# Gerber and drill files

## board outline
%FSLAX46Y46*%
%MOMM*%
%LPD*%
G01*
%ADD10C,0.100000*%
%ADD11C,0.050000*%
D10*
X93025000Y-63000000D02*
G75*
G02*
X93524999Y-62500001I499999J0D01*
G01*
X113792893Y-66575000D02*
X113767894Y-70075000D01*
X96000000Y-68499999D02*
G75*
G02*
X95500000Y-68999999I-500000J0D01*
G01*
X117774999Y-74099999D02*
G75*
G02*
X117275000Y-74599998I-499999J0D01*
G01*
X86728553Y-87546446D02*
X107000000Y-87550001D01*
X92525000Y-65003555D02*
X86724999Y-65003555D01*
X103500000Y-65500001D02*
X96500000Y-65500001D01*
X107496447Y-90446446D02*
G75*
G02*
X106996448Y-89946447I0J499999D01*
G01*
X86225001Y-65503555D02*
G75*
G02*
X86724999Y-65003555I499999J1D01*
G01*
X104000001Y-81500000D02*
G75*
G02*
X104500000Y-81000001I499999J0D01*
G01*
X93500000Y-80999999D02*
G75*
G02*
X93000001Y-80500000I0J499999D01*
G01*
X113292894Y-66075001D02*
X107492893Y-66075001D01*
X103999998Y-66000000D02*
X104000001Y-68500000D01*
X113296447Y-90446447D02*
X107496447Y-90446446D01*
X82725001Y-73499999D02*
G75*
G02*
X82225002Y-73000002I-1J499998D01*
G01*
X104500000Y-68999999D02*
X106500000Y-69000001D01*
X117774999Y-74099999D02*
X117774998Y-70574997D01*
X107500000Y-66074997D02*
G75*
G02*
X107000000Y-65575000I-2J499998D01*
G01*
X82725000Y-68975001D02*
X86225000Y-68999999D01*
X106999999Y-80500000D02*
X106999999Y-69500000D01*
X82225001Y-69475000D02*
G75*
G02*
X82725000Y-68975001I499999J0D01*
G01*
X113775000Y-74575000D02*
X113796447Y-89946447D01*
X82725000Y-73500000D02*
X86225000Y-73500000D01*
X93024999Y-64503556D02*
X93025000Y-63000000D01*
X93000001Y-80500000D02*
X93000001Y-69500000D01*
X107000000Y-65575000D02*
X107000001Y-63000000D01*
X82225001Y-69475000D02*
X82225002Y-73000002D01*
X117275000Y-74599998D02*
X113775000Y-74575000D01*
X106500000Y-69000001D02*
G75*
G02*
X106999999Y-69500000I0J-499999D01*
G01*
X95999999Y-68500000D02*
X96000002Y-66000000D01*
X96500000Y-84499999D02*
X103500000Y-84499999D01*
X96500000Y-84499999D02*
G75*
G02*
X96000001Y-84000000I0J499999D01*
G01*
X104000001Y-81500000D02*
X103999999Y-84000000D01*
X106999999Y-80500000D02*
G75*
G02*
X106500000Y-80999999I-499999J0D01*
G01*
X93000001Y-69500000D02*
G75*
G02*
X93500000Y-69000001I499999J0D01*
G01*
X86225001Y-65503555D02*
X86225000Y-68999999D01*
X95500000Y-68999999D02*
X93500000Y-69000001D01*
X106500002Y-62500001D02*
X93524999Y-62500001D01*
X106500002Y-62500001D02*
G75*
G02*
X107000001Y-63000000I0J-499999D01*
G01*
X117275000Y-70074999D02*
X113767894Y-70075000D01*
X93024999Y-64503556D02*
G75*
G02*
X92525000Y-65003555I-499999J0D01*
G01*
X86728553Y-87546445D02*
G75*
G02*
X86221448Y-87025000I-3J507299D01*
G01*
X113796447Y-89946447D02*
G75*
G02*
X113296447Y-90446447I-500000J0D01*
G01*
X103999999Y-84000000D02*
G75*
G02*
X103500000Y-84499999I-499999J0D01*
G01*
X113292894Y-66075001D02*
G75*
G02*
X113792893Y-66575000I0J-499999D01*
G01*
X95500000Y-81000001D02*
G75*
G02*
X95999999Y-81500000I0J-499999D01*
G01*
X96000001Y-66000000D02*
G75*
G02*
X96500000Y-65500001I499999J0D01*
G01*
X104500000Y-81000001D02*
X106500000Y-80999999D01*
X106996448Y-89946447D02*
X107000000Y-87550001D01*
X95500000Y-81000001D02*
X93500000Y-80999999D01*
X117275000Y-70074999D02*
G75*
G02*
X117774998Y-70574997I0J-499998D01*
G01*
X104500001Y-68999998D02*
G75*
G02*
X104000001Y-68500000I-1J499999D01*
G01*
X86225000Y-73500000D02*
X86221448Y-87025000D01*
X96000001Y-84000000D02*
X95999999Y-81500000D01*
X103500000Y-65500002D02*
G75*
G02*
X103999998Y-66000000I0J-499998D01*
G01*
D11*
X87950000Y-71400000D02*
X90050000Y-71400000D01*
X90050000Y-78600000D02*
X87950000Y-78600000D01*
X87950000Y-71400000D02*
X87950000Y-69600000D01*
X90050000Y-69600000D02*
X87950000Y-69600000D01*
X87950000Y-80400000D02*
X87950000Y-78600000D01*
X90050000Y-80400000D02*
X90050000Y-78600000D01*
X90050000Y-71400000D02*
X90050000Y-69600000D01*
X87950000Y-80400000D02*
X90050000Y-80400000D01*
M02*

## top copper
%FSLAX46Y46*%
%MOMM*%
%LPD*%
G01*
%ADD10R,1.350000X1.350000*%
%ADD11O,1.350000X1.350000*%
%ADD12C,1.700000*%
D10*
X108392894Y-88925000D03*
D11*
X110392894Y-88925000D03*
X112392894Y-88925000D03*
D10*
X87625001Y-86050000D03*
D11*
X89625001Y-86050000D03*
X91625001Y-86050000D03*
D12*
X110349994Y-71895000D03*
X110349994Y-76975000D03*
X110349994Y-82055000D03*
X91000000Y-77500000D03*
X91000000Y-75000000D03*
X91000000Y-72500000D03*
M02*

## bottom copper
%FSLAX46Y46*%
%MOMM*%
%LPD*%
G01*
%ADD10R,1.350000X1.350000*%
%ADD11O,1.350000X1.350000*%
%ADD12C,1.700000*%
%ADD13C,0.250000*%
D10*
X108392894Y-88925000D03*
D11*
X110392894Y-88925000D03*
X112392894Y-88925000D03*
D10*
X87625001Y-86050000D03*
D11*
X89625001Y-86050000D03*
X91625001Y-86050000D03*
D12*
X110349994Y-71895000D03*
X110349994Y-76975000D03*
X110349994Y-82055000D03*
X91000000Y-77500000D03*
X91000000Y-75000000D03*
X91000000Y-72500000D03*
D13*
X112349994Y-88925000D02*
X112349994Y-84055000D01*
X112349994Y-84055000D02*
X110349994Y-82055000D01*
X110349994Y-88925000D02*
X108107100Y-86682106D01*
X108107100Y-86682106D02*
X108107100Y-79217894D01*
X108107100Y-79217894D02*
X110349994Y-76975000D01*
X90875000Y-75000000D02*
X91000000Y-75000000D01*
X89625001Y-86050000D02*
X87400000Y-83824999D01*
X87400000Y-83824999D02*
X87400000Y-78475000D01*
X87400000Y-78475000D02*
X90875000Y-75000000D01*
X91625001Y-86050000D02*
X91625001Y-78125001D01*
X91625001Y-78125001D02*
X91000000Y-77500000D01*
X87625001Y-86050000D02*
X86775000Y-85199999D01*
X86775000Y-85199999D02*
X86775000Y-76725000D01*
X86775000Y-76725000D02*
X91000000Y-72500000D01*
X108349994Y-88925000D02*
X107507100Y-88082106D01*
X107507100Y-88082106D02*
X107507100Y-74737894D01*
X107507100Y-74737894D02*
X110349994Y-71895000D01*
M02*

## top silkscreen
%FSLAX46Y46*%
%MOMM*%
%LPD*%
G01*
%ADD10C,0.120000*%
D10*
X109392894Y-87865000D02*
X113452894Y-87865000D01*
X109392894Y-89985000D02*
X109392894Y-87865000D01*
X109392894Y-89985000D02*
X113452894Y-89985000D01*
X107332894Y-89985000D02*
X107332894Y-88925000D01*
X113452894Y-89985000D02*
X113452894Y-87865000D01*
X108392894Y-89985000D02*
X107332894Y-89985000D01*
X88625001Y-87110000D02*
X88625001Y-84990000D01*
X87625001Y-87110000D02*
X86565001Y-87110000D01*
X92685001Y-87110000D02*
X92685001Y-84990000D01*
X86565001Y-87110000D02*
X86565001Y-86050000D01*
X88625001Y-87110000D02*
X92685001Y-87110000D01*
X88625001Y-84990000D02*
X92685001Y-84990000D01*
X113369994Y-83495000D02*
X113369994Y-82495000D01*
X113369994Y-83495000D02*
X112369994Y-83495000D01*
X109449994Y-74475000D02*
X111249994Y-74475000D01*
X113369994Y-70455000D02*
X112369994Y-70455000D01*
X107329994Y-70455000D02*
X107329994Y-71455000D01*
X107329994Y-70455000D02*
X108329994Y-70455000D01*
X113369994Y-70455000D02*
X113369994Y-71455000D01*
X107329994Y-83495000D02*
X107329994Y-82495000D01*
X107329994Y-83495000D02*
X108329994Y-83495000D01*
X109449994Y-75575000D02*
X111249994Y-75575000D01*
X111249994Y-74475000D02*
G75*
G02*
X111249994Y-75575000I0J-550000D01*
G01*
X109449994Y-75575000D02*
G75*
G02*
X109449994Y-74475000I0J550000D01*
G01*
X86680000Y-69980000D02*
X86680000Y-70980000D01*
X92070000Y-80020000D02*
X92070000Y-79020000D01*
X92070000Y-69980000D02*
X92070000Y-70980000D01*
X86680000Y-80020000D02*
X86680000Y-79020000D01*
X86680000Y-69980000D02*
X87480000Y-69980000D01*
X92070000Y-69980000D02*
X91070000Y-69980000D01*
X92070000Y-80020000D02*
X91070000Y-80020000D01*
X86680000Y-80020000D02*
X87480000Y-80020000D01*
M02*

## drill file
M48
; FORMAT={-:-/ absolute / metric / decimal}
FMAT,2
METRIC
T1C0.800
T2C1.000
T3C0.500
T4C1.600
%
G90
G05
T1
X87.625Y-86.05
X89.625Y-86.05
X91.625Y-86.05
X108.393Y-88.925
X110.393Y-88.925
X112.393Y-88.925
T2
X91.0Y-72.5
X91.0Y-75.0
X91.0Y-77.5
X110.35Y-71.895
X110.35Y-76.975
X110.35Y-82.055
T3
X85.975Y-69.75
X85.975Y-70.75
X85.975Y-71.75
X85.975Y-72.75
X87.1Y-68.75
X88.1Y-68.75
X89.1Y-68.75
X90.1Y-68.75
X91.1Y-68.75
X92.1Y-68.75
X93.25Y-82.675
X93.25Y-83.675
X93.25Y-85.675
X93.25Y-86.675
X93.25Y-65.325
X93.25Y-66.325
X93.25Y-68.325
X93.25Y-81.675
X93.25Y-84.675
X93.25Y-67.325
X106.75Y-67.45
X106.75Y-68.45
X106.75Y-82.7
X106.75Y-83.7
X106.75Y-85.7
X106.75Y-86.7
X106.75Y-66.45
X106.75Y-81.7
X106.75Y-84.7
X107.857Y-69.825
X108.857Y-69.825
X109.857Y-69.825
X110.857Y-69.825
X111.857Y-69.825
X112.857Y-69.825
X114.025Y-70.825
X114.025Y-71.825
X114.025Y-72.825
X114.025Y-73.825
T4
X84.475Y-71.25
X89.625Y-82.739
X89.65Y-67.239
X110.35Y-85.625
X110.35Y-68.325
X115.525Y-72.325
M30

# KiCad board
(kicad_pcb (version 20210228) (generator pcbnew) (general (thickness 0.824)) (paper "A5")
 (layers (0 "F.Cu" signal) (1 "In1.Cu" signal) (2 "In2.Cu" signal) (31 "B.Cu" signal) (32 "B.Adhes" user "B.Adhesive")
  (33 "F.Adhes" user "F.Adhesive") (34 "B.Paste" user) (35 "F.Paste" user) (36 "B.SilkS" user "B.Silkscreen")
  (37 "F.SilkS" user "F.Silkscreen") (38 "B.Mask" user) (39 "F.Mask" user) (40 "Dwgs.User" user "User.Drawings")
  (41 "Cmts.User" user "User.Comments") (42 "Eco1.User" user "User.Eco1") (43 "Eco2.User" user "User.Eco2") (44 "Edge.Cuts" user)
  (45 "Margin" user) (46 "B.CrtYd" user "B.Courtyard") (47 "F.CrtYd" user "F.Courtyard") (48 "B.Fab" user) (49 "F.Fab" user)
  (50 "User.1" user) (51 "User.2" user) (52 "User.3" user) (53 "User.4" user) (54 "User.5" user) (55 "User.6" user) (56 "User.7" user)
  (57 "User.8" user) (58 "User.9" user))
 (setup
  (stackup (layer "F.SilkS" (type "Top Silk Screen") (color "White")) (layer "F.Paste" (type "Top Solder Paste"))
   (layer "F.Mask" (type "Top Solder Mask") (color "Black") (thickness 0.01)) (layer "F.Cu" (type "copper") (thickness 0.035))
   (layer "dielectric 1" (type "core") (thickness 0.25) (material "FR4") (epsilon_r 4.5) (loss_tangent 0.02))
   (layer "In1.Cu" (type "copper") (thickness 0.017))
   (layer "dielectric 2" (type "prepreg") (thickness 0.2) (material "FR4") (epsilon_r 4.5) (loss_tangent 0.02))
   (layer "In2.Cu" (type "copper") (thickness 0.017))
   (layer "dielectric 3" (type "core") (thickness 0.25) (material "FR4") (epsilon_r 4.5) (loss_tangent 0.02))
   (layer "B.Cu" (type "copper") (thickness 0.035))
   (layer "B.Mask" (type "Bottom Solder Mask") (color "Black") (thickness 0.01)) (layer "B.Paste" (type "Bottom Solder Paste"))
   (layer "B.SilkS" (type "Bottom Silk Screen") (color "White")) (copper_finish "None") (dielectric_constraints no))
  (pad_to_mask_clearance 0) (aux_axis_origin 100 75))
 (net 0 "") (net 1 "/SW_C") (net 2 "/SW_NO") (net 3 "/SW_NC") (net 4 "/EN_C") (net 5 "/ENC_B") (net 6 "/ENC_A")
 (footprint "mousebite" (layer "F.Cu") (at 112.8571 69.824999 -90)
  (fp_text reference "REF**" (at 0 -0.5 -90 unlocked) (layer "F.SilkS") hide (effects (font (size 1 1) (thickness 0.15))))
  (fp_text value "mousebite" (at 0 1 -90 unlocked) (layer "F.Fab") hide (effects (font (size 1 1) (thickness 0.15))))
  (pad "" np_thru_hole circle (at 0 0 270) (size 0.5 0.5) (drill 0.5) (layers F&B.Cu *.Mask)))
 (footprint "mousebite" (layer "F.Cu") (at 93.249999 82.675001 180)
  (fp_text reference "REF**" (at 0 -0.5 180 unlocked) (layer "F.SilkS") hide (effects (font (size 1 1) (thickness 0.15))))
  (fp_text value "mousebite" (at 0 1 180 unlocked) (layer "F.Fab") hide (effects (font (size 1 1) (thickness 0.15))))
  (pad "" np_thru_hole circle (at 0 0 180) (size 0.5 0.5) (drill 0.5) (layers F&B.Cu *.Mask)))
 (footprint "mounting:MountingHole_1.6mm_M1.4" (layer "F.Cu") (at 89.650001 67.239304 -90)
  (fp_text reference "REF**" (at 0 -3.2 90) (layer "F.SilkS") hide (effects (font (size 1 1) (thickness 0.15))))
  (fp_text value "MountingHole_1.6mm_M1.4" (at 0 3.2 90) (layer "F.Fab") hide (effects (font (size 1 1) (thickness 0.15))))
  (pad "" np_thru_hole circle (at 0 0 270) (locked) (size 1.6 1.6) (drill 1.6) (layers F&B.Cu *.Mask)))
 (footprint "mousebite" (layer "F.Cu") (at 110.8571 69.824999 -90)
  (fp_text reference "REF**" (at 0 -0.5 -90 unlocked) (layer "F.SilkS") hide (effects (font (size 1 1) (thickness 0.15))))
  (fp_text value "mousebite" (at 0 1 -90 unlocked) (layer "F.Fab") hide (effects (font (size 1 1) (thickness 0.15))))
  (pad "" np_thru_hole circle (at 0 0 270) (size 0.5 0.5) (drill 0.5) (layers F&B.Cu *.Mask)))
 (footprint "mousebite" (layer "F.Cu") (at 106.749999 67.45 180)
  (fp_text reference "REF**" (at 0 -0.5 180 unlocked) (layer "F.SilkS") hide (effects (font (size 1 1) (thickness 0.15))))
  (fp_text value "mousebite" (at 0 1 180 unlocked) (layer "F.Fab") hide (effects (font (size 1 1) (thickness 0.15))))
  (pad "" np_thru_hole circle (at 0 0 180) (size 0.5 0.5) (drill 0.5) (layers F&B.Cu *.Mask)))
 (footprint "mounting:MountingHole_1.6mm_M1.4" (layer "F.Cu") (at 110.349995 68.325 -90)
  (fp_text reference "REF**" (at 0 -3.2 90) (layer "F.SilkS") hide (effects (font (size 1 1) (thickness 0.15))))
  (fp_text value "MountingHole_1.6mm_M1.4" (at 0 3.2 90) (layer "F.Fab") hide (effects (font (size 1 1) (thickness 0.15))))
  (pad "" np_thru_hole circle (at 0 0 270) (locked) (size 1.6 1.6) (drill 1.6) (layers F&B.Cu *.Mask)))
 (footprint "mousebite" (layer "F.Cu") (at 85.975 72.749998)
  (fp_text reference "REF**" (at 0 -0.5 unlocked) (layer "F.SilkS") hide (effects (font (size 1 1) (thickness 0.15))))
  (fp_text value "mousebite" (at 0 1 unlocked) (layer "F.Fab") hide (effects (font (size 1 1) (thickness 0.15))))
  (pad "" np_thru_hole circle (at 0 0) (size 0.5 0.5) (drill 0.5) (layers F&B.Cu *.Mask)))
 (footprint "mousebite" (layer "F.Cu") (at 93.249999 83.675 180)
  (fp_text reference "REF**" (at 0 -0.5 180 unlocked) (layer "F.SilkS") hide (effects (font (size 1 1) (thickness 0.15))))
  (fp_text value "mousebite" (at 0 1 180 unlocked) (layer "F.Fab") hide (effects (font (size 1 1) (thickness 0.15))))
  (pad "" np_thru_hole circle (at 0 0 180) (size 0.5 0.5) (drill 0.5) (layers F&B.Cu *.Mask)))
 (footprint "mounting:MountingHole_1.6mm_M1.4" (layer "F.Cu") (at 89.625 82.73925 -90)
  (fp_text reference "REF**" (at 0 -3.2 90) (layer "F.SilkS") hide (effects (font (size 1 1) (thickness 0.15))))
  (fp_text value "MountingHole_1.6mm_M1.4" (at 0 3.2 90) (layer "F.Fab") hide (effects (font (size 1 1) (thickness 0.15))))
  (pad "" np_thru_hole circle (at 0 0 270) (locked) (size 1.6 1.6) (drill 1.6) (layers F&B.Cu *.Mask)))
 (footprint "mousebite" (layer "F.Cu") (at 108.8571 69.824999 -90)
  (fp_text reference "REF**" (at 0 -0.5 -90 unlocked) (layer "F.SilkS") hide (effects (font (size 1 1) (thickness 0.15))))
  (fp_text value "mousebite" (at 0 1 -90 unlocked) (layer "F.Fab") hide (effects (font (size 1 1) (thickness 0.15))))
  (pad "" np_thru_hole circle (at 0 0 270) (size 0.5 0.5) (drill 0.5) (layers F&B.Cu *.Mask)))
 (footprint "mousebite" (layer "F.Cu") (at 88.1 68.75 90)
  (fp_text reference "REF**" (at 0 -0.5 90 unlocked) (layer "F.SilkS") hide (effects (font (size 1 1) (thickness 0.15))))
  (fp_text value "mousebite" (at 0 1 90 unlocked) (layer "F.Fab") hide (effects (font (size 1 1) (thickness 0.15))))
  (pad "" np_thru_hole circle (at 0 0 90) (size 0.5 0.5) (drill 0.5) (layers F&B.Cu *.Mask)))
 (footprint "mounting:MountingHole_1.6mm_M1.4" (layer "F.Cu") (at 84.475001 71.25)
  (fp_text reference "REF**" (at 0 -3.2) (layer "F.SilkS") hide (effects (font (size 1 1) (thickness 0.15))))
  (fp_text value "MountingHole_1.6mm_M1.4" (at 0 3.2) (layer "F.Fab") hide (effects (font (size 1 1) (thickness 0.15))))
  (pad "" np_thru_hole circle (at 0 0) (locked) (size 1.6 1.6) (drill 1.6) (layers F&B.Cu *.Mask)))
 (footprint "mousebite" (layer "F.Cu") (at 106.75 81.700001 180)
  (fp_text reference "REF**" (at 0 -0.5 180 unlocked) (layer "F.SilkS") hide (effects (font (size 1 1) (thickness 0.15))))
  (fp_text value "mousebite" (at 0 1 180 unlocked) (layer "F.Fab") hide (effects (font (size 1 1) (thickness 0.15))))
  (pad "" np_thru_hole circle (at 0 0 180) (size 0.5 0.5) (drill 0.5) (layers F&B.Cu *.Mask)))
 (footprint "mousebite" (layer "F.Cu") (at 111.8571 69.824999 -90)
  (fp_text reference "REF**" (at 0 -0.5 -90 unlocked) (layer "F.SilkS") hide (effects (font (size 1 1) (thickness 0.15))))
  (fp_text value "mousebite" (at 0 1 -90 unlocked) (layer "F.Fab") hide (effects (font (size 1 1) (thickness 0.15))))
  (pad "" np_thru_hole circle (at 0 0 270) (size 0.5 0.5) (drill 0.5) (layers F&B.Cu *.Mask)))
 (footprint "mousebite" (layer "F.Cu") (at 90.1 68.75 90)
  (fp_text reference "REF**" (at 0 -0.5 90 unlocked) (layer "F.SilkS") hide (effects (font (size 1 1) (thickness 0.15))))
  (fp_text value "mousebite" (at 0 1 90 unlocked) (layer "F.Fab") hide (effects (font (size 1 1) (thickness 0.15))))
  (pad "" np_thru_hole circle (at 0 0 90) (size 0.5 0.5) (drill 0.5) (layers F&B.Cu *.Mask)))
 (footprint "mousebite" (layer "F.Cu") (at 85.975 71.749999)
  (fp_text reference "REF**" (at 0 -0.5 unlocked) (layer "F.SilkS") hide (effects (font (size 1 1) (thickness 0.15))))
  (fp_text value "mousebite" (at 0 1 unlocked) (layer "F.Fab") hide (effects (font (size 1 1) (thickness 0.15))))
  (pad "" np_thru_hole circle (at 0 0) (size 0.5 0.5) (drill 0.5) (layers F&B.Cu *.Mask)))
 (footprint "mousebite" (layer "F.Cu") (at 106.75 84.700001 180)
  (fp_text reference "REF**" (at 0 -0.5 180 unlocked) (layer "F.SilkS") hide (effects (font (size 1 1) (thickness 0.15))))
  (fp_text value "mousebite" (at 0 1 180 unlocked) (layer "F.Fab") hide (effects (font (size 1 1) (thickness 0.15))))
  (pad "" np_thru_hole circle (at 0 0 180) (size 0.5 0.5) (drill 0.5) (layers F&B.Cu *.Mask)))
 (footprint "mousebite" (layer "F.Cu") (at 87.1 68.75 90)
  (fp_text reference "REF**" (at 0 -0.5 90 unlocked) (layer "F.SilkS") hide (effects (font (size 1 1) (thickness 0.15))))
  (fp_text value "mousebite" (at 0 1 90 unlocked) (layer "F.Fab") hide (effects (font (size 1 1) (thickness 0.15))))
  (pad "" np_thru_hole circle (at 0 0 90) (size 0.5 0.5) (drill 0.5) (layers F&B.Cu *.Mask)))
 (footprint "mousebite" (layer "F.Cu") (at 114.025 70.825001 180)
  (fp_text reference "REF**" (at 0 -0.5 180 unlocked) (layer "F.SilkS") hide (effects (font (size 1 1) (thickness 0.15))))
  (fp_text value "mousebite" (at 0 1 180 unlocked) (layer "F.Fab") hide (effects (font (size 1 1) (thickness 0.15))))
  (pad "" np_thru_hole circle (at 0 0 180) (size 0.5 0.5) (drill 0.5) (layers F&B.Cu *.Mask)))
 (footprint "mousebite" (layer "F.Cu") (at 106.749999 86.7 180)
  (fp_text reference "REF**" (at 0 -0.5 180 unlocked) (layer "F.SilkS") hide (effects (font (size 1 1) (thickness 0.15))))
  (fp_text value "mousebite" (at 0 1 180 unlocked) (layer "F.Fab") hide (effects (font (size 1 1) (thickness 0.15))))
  (pad "" np_thru_hole circle (at 0 0 180) (size 0.5 0.5) (drill 0.5) (layers F&B.Cu *.Mask)))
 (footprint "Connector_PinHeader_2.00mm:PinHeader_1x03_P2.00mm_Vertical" (layer "F.Cu") (at 108.392894 88.925 90)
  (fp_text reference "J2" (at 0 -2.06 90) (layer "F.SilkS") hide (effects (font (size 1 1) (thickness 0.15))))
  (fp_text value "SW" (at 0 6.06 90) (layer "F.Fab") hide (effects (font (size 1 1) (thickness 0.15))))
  (fp_line (start 1.06 1) (end 1.06 5.06) (layer "F.SilkS") (width 0.12))
  (fp_line (start -1.06 1) (end 1.06 1) (layer "F.SilkS") (width 0.12))
  (fp_line (start -1.06 1) (end -1.06 5.06) (layer "F.SilkS") (width 0.12))
  (fp_line (start -1.06 -1.06) (end 0 -1.06) (layer "F.SilkS") (width 0.12))
  (fp_line (start -1.06 5.06) (end 1.06 5.06) (layer "F.SilkS") (width 0.12))
  (fp_line (start -1.06 0) (end -1.06 -1.06) (layer "F.SilkS") (width 0.12))
  (pad "1" thru_hole rect (at 0 0 90) (locked) (size 1.35 1.35) (drill 0.8) (layers *.Cu *.Mask) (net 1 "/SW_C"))
  (pad "2" thru_hole oval (at 0 2 90) (locked) (size 1.35 1.35) (drill 0.8) (layers *.Cu *.Mask) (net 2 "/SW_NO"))
  (pad "3" thru_hole oval (at 0 4 90) (locked) (size 1.35 1.35) (drill 0.8) (layers *.Cu *.Mask) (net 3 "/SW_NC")))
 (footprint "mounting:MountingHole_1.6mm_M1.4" (layer "F.Cu") (at 110.349994 85.625 -90)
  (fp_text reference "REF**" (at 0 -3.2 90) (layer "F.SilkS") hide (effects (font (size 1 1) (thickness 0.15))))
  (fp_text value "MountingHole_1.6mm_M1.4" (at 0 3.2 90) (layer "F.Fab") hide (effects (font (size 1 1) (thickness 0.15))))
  (pad "" np_thru_hole circle (at 0 0 270) (locked) (size 1.6 1.6) (drill 1.6) (layers F&B.Cu *.Mask)))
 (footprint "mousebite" (layer "F.Cu") (at 92.1 68.75 90)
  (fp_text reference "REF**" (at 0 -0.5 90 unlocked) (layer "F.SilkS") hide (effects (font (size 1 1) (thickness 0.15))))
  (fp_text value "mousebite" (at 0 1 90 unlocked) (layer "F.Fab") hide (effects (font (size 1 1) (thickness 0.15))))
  (pad "" np_thru_hole circle (at 0 0 90) (size 0.5 0.5) (drill 0.5) (layers F&B.Cu *.Mask)))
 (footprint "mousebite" (layer "F.Cu") (at 93.25 66.324999 180)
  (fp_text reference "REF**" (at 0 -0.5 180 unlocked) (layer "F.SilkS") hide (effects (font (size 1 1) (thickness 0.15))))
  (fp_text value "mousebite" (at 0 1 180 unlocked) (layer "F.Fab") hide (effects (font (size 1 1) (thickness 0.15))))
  (pad "" np_thru_hole circle (at 0 0 180) (size 0.5 0.5) (drill 0.5) (layers F&B.Cu *.Mask)))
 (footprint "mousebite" (layer "F.Cu") (at 93.25 84.675001 180)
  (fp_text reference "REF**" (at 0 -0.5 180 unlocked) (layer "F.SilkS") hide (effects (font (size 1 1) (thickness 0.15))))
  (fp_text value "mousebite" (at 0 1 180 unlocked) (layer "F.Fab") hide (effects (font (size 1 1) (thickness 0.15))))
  (pad "" np_thru_hole circle (at 0 0 180) (size 0.5 0.5) (drill 0.5) (layers F&B.Cu *.Mask)))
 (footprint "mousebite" (layer "F.Cu") (at 106.749999 68.449999 180)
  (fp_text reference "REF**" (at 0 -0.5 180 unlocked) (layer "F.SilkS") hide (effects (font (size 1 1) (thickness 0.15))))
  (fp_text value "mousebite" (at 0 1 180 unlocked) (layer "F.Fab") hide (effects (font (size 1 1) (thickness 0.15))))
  (pad "" np_thru_hole circle (at 0 0 180) (size 0.5 0.5) (drill 0.5) (layers F&B.Cu *.Mask)))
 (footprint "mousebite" (layer "F.Cu") (at 93.249999 86.675 180)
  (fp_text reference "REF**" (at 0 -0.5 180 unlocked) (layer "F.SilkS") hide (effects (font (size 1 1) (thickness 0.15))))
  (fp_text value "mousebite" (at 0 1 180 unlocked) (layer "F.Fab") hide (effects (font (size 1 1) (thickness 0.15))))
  (pad "" np_thru_hole circle (at 0 0 180) (size 0.5 0.5) (drill 0.5) (layers F&B.Cu *.Mask)))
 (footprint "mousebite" (layer "F.Cu") (at 106.749999 85.700001 180)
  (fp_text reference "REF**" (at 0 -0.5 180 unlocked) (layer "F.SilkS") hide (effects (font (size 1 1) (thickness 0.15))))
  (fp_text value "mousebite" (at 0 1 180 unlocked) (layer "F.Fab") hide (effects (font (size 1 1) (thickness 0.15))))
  (pad "" np_thru_hole circle (at 0 0 180) (size 0.5 0.5) (drill 0.5) (layers F&B.Cu *.Mask)))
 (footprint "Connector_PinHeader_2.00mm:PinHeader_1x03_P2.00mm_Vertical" (layer "F.Cu") (at 87.625001 86.05 90)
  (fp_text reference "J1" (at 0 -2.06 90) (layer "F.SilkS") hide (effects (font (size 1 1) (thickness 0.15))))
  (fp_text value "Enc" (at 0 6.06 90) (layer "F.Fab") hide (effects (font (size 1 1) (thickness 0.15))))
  (fp_line (start -1.06 1) (end 1.06 1) (layer "F.SilkS") (width 0.12))
  (fp_line (start -1.06 0) (end -1.06 -1.06) (layer "F.SilkS") (width 0.12))
  (fp_line (start -1.06 5.06) (end 1.06 5.06) (layer "F.SilkS") (width 0.12))
  (fp_line (start -1.06 -1.06) (end 0 -1.06) (layer "F.SilkS") (width 0.12))
  (fp_line (start -1.06 1) (end -1.06 5.06) (layer "F.SilkS") (width 0.12))
  (fp_line (start 1.06 1) (end 1.06 5.06) (layer "F.SilkS") (width 0.12))
  (pad "1" thru_hole rect (at 0 0 90) (locked) (size 1.35 1.35) (drill 0.8) (layers *.Cu *.Mask) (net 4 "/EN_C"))
  (pad "2" thru_hole oval (at 0 2 90) (locked) (size 1.35 1.35) (drill 0.8) (layers *.Cu *.Mask) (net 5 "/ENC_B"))
  (pad "3" thru_hole oval (at 0 4 90) (locked) (size 1.35 1.35) (drill 0.8) (layers *.Cu *.Mask) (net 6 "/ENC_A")))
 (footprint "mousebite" (layer "F.Cu") (at 106.75 66.45 180)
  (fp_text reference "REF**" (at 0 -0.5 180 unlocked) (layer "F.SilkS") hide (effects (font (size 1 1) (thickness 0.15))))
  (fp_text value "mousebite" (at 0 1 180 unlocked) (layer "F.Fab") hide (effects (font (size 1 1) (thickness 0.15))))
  (pad "" np_thru_hole circle (at 0 0 180) (size 0.5 0.5) (drill 0.5) (layers F&B.Cu *.Mask)))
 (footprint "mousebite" (layer "F.Cu") (at 107.8571 69.824999 -90)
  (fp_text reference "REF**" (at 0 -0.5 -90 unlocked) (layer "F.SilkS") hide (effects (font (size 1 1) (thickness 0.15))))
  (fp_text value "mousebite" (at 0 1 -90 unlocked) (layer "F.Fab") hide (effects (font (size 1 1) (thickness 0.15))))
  (pad "" np_thru_hole circle (at 0 0 270) (size 0.5 0.5) (drill 0.5) (layers F&B.Cu *.Mask)))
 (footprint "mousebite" (layer "F.Cu") (at 85.975 69.750002)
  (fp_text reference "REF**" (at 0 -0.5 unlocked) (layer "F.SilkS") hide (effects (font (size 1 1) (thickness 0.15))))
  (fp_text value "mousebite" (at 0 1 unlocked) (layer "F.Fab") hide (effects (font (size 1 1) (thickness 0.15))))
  (pad "" np_thru_hole circle (at 0 0) (size 0.5 0.5) (drill 0.5) (layers F&B.Cu *.Mask)))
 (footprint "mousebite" (layer "F.Cu") (at 93.25 65.325 180)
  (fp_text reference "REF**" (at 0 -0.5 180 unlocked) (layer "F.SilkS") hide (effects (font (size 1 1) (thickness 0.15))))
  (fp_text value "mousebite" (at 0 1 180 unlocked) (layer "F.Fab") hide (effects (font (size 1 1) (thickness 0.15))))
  (pad "" np_thru_hole circle (at 0 0 180) (size 0.5 0.5) (drill 0.5) (layers F&B.Cu *.Mask)))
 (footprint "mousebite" (layer "F.Cu") (at 85.975 70.750001)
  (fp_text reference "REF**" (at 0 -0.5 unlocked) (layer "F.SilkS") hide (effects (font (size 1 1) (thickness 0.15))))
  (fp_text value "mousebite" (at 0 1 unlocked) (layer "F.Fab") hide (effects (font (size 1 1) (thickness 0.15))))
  (pad "" np_thru_hole circle (at 0 0) (size 0.5 0.5) (drill 0.5) (layers F&B.Cu *.Mask)))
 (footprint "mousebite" (layer "F.Cu") (at 93.25 68.325 180)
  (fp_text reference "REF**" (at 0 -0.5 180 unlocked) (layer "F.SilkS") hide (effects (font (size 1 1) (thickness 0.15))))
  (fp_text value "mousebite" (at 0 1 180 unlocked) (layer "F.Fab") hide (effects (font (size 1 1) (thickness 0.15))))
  (pad "" np_thru_hole circle (at 0 0 180) (size 0.5 0.5) (drill 0.5) (layers F&B.Cu *.Mask)))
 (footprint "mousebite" (layer "F.Cu") (at 93.250001 67.325 180)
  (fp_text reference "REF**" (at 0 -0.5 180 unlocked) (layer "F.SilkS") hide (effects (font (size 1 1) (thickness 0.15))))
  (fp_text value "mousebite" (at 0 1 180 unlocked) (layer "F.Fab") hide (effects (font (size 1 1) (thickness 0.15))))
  (pad "" np_thru_hole circle (at 0 0 180) (size 0.5 0.5) (drill 0.5) (layers F&B.Cu *.Mask)))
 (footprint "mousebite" (layer "F.Cu") (at 114.025 71.825 180)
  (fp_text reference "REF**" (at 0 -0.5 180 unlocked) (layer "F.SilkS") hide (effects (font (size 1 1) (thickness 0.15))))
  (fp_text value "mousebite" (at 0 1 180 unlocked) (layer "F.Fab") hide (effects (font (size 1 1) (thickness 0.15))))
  (pad "" np_thru_hole circle (at 0 0 180) (size 0.5 0.5) (drill 0.5) (layers F&B.Cu *.Mask)))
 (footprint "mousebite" (layer "F.Cu") (at 91.1 68.75 90)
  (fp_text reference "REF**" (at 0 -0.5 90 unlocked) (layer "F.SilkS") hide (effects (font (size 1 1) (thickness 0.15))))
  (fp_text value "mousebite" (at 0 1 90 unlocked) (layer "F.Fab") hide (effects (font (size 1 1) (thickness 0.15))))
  (pad "" np_thru_hole circle (at 0 0 90) (size 0.5 0.5) (drill 0.5) (layers F&B.Cu *.Mask)))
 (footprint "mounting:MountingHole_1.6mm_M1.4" (layer "F.Cu") (at 115.524999 72.324999 180)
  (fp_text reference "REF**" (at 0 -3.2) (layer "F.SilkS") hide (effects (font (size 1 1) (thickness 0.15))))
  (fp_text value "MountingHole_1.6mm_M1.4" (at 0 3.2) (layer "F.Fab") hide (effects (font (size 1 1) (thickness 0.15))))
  (pad "" np_thru_hole circle (at 0 0 180) (locked) (size 1.6 1.6) (drill 1.6) (layers F&B.Cu *.Mask)))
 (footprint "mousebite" (layer "F.Cu") (at 106.749999 83.7 180)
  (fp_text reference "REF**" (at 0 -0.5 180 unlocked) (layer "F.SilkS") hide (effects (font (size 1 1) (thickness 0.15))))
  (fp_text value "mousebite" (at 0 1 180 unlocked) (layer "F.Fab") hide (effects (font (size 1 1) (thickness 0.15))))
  (pad "" np_thru_hole circle (at 0 0 180) (size 0.5 0.5) (drill 0.5) (layers F&B.Cu *.Mask)))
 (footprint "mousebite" (layer "F.Cu") (at 93.249999 85.675001 180)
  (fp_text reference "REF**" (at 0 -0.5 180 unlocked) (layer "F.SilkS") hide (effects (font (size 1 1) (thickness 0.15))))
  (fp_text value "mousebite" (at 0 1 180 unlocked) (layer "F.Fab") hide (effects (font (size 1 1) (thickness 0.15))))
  (pad "" np_thru_hole circle (at 0 0 180) (size 0.5 0.5) (drill 0.5) (layers F&B.Cu *.Mask)))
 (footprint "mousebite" (layer "F.Cu") (at 114.025 72.824998 180)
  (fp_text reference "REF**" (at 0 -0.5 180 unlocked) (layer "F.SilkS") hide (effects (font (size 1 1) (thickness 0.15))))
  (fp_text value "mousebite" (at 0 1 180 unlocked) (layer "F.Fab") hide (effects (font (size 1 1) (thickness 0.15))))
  (pad "" np_thru_hole circle (at 0 0 180) (size 0.5 0.5) (drill 0.5) (layers F&B.Cu *.Mask)))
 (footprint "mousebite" (layer "F.Cu") (at 114.025 73.824997 180)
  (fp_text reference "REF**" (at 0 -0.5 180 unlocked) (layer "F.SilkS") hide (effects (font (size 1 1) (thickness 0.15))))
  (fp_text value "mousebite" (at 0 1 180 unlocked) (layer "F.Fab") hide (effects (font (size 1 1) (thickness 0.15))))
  (pad "" np_thru_hole circle (at 0 0 180) (size 0.5 0.5) (drill 0.5) (layers F&B.Cu *.Mask)))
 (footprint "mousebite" (layer "F.Cu") (at 89.1 68.75 90)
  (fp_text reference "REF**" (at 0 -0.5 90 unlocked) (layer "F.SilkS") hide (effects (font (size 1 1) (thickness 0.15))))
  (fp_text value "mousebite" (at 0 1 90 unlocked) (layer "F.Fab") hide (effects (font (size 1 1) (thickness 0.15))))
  (pad "" np_thru_hole circle (at 0 0 90) (size 0.5 0.5) (drill 0.5) (layers F&B.Cu *.Mask)))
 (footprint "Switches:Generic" (layer "F.Cu") (at 110.349994 76.975 -90)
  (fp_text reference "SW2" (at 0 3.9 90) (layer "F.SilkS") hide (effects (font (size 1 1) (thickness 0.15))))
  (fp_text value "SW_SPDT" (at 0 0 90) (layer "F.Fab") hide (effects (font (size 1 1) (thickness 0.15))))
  (fp_line (start 6.52 -3.02) (end 5.52 -3.02) (layer "F.SilkS") (width 0.12))
  (fp_line (start 6.52 -3.02) (end 6.52 -2.02) (layer "F.SilkS") (width 0.12))
  (fp_line (start -2.5 0.9) (end -2.5 -0.9) (layer "F.SilkS") (width 0.12))
  (fp_line (start -6.52 -3.02) (end -6.52 -2.02) (layer "F.SilkS") (width 0.12))
  (fp_line (start -6.52 3.02) (end -5.52 3.02) (layer "F.SilkS") (width 0.12))
  (fp_line (start -6.52 3.02) (end -6.52 2.02) (layer "F.SilkS") (width 0.12))
  (fp_line (start -6.52 -3.02) (end -5.52 -3.02) (layer "F.SilkS") (width 0.12))
  (fp_line (start 6.52 3.02) (end 5.52 3.02) (layer "F.SilkS") (width 0.12))
  (fp_line (start 6.52 3.02) (end 6.52 2.02) (layer "F.SilkS") (width 0.12))
  (fp_line (start -1.4 0.9) (end -1.4 -0.9) (layer "F.SilkS") (width 0.12))
  (fp_arc (start -1.95 -0.9) (end -1.4 -0.9) (angle -180) (layer "F.SilkS") (width 0.12))
  (fp_arc (start -1.95 0.9) (end -2.5 0.9) (angle -180) (layer "F.SilkS") (width 0.12))
  (pad "1" thru_hole circle (at -5.08 0 270) (locked) (size 1.7 1.7) (drill 1) (layers *.Cu *.Mask) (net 1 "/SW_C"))
  (pad "2" thru_hole circle (at 0 0 270) (locked) (size 1.7 1.7) (drill 1) (layers *.Cu *.Mask) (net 2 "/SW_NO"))
  (pad "3" thru_hole circle (at 5.08 0 270) (locked) (size 1.7 1.7) (drill 1) (layers *.Cu *.Mask) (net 3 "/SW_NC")))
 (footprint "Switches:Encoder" (layer "F.Cu") (at 91 75 90)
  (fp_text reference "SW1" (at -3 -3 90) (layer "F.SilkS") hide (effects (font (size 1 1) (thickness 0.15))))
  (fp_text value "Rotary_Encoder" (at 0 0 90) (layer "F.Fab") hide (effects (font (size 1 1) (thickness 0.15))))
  (fp_line (start 5.02 -4.32) (end 4.02 -4.32) (layer "F.SilkS") (width 0.12))
  (fp_line (start -5.02 1.07) (end -4.02 1.07) (layer "F.SilkS") (width 0.12))
  (fp_line (start 5.02 1.07) (end 4.02 1.07) (layer "F.SilkS") (width 0.12))
  (fp_line (start -5.02 -4.32) (end -4.02 -4.32) (layer "F.SilkS") (width 0.12))
  (fp_line (start 5.02 -4.32) (end 5.02 -3.52) (layer "F.SilkS") (width 0.12))
  (fp_line (start 5.02 1.07) (end 5.02 0.07) (layer "F.SilkS") (width 0.12))
  (fp_line (start -5.02 1.07) (end -5.02 0.07) (layer "F.SilkS") (width 0.12))
  (fp_line (start -5.02 -4.32) (end -5.02 -3.52) (layer "F.SilkS") (width 0.12))
  (fp_line (start 3.6 -3.05) (end 3.6 -0.95) (layer "Edge.Cuts") (width 0.05))
  (fp_line (start -3.6 -0.95) (end -3.6 -3.05) (layer "Edge.Cuts") (width 0.05))
  (fp_line (start 3.6 -3.05) (end 5.4 -3.05) (layer "Edge.Cuts") (width 0.05))
  (fp_line (start 5.4 -0.95) (end 5.4 -3.05) (layer "Edge.Cuts") (width 0.05))
  (fp_line (start -5.4 -3.05) (end -3.6 -3.05) (layer "Edge.Cuts") (width 0.05))
  (fp_line (start -5.4 -0.95) (end -3.6 -0.95) (layer "Edge.Cuts") (width 0.05))
  (fp_line (start 3.6 -0.95) (end 5.4 -0.95) (layer "Edge.Cuts") (width 0.05))
  (fp_line (start -5.4 -3.05) (end -5.4 -0.95) (layer "Edge.Cuts") (width 0.05))
  (pad "A" thru_hole circle (at -2.5 0 90) (locked) (size 1.7 1.7) (drill 1) (layers *.Cu *.Mask) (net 6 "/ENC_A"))
  (pad "B" thru_hole circle (at 0 0 90) (locked) (size 1.7 1.7) (drill 1) (layers *.Cu *.Mask) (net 5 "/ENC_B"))
  (pad "C" thru_hole circle (at 2.5 0 90) (locked) (size 1.7 1.7) (drill 1) (layers *.Cu *.Mask) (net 4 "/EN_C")))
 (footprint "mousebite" (layer "F.Cu") (at 93.25 81.675001 180)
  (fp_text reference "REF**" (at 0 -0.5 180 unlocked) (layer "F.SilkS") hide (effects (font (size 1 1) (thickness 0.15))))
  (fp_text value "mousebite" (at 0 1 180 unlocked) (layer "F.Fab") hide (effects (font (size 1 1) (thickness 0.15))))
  (pad "" np_thru_hole circle (at 0 0 180) (size 0.5 0.5) (drill 0.5) (layers F&B.Cu *.Mask)))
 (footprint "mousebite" (layer "F.Cu") (at 106.749999 82.700001 180)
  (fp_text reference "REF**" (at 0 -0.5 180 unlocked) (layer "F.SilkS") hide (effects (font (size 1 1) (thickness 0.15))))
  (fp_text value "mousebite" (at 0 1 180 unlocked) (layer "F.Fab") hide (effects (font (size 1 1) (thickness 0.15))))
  (pad "" np_thru_hole circle (at 0 0 180) (size 0.5 0.5) (drill 0.5) (layers F&B.Cu *.Mask)))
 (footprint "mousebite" (layer "F.Cu") (at 109.8571 69.824999 -90)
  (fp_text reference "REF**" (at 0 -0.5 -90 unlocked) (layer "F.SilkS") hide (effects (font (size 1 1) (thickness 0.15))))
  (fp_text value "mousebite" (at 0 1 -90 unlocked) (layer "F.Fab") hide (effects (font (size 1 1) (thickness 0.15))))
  (pad "" np_thru_hole circle (at 0 0 270) (size 0.5 0.5) (drill 0.5) (layers F&B.Cu *.Mask)))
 (gr_arc (start 93.524999 63) (end 93.524999 62.500001) (angle -90) (layer "Edge.Cuts") (width 0.1))
 (gr_line (start 113.792893 66.575) (end 113.767894 70.075) (layer "Edge.Cuts") (width 0.1))
 (gr_arc (start 95.5 68.499999) (end 95.5 68.999999) (angle -90) (layer "Edge.Cuts") (width 0.1))
 (gr_arc (start 117.275 74.099999) (end 117.275 74.599998) (angle -90) (layer "Edge.Cuts") (width 0.1))
 (gr_line (start 86.728553 87.546446) (end 107 87.550001) (layer "Edge.Cuts") (width 0.1))
 (gr_line (start 92.525 65.003555) (end 86.724999 65.003555) (layer "Edge.Cuts") (width 0.1))
 (gr_line (start 103.5 65.500001) (end 96.5 65.500001) (layer "Edge.Cuts") (width 0.1))
 (gr_arc (start 107.496447 89.946447) (end 106.996448 89.946447) (angle -90) (layer "Edge.Cuts") (width 0.1))
 (gr_arc (start 86.725 65.503554) (end 86.724999 65.003555) (angle -90) (layer "Edge.Cuts") (width 0.1))
 (gr_arc (start 104.5 81.5) (end 104.5 81.000001) (angle -90) (layer "Edge.Cuts") (width 0.1))
 (gr_arc (start 93.5 80.5) (end 93.000001 80.5) (angle -90) (layer "Edge.Cuts") (width 0.1))
 (gr_line (start 113.292894 66.075001) (end 107.492893 66.075001) (layer "Edge.Cuts") (width 0.1))
 (gr_line (start 103.999998 66) (end 104.000001 68.5) (layer "Edge.Cuts") (width 0.1))
 (gr_line (start 113.296447 90.446447) (end 107.496447 90.446446) (layer "Edge.Cuts") (width 0.1))
 (gr_arc (start 82.725 73.000001) (end 82.225002 73.000002) (angle -90) (layer "Edge.Cuts") (width 0.1))
 (gr_line (start 104.5 68.999999) (end 106.5 69.000001) (layer "Edge.Cuts") (width 0.1))
 (gr_line (start 117.774999 74.099999) (end 117.774998 70.574997) (layer "Edge.Cuts") (width 0.1))
 (gr_arc (start 107.499998 65.574999) (end 107 65.575) (angle -90.00011459) (layer "Edge.Cuts") (width 0.1))
 (gr_line (start 82.725 68.975001) (end 86.225 68.999999) (layer "Edge.Cuts") (width 0.1))
 (gr_line (start 106.999999 80.5) (end 106.999999 69.5) (layer "Edge.Cuts") (width 0.1))
 (gr_arc (start 82.725 69.475) (end 82.725 68.975001) (angle -90) (layer "Edge.Cuts") (width 0.1))
 (gr_line (start 113.775 74.575) (end 113.796447 89.946447) (layer "Edge.Cuts") (width 0.1))
 (gr_line (start 82.725 73.5) (end 86.225 73.5) (layer "Edge.Cuts") (width 0.1))
 (gr_line (start 93.024999 64.503556) (end 93.025 63) (layer "Edge.Cuts") (width 0.1))
 (gr_line (start 93.000001 80.5) (end 93.000001 69.5) (layer "Edge.Cuts") (width 0.1))
 (gr_line (start 107 65.575) (end 107.000001 63) (layer "Edge.Cuts") (width 0.1))
 (gr_line (start 82.225001 69.475) (end 82.225002 73.000002) (layer "Edge.Cuts") (width 0.1))
 (gr_line (start 117.275 74.599998) (end 113.775 74.575) (layer "Edge.Cuts") (width 0.1))
 (gr_arc (start 106.5 69.5) (end 106.999999 69.5) (angle -90) (layer "Edge.Cuts") (width 0.1))
 (gr_line (start 95.999999 68.5) (end 96.000002 66) (layer "Edge.Cuts") (width 0.1))
 (gr_line (start 96.5 84.499999) (end 103.5 84.499999) (layer "Edge.Cuts") (width 0.1))
 (gr_arc (start 96.5 84) (end 96.000001 84) (angle -90) (layer "Edge.Cuts") (width 0.1))
 (gr_line (start 104.000001 81.5) (end 103.999999 84) (layer "Edge.Cuts") (width 0.1))
 (gr_arc (start 106.5 80.5) (end 106.5 80.999999) (angle -90) (layer "Edge.Cuts") (width 0.1))
 (gr_arc (start 93.5 69.5) (end 93.5 69.000001) (angle -90) (layer "Edge.Cuts") (width 0.1))
 (gr_line (start 86.225001 65.503555) (end 86.225 68.999999) (layer "Edge.Cuts") (width 0.1))
 (gr_line (start 95.5 68.999999) (end 93.5 69.000001) (layer "Edge.Cuts") (width 0.1))
 (gr_line (start 106.500002 62.500001) (end 93.524999 62.500001) (layer "Edge.Cuts") (width 0.1))
 (gr_arc (start 106.500002 63) (end 107.000001 63) (angle -90) (layer "Edge.Cuts") (width 0.1))
 (gr_line (start 117.275 70.074999) (end 113.767894 70.075) (layer "Edge.Cuts") (width 0.1))
 (gr_arc (start 92.525 64.503556) (end 92.525 65.003555) (angle -90) (layer "Edge.Cuts") (width 0.1))
 (gr_arc (start 86.72855 87.039146) (end 86.221448 87.025) (angle -91.59823424) (layer "Edge.Cuts") (width 0.1))
 (gr_arc (start 113.296447 89.946447) (end 113.296447 90.446447) (angle -90) (layer "Edge.Cuts") (width 0.1))
 (gr_arc (start 103.5 84) (end 103.5 84.499999) (angle -90) (layer "Edge.Cuts") (width 0.1))
 (gr_arc (start 113.292894 66.575) (end 113.792893 66.575) (angle -90) (layer "Edge.Cuts") (width 0.1))
 (gr_arc (start 95.5 81.5) (end 95.999999 81.5) (angle -90) (layer "Edge.Cuts") (width 0.1))
 (gr_arc (start 96.5 66) (end 96.5 65.500001) (angle -90) (layer "Edge.Cuts") (width 0.1))
 (gr_line (start 104.5 81.000001) (end 106.5 80.999999) (layer "Edge.Cuts") (width 0.1))
 (gr_line (start 106.996448 89.946447) (end 107 87.550001) (layer "Edge.Cuts") (width 0.1))
 (gr_line (start 95.5 81.000001) (end 93.5 80.999999) (layer "Edge.Cuts") (width 0.1))
 (gr_arc (start 117.275 70.574997) (end 117.774998 70.574997) (angle -90) (layer "Edge.Cuts") (width 0.1))
 (gr_arc (start 104.5 68.499999) (end 104.000001 68.5) (angle -90) (layer "Edge.Cuts") (width 0.1))
 (gr_line (start 86.225 73.5) (end 86.221448 87.025) (layer "Edge.Cuts") (width 0.1))
 (gr_line (start 96.000001 84) (end 95.999999 81.5) (layer "Edge.Cuts") (width 0.1))
 (gr_arc (start 103.5 66) (end 103.999998 66) (angle -90) (layer "Edge.Cuts") (width 0.1))
 (segment (start 112.349994 88.925) (end 112.349994 84.055) (width 0.25) (layer "B.Cu") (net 3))
 (segment (start 112.349994 84.055) (end 110.349994 82.055) (width 0.25) (layer "B.Cu") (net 3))
 (segment (start 110.349994 88.925) (end 108.1071 86.682106) (width 0.25) (layer "B.Cu") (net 2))
 (segment (start 108.1071 86.682106) (end 108.1071 79.217894) (width 0.25) (layer "B.Cu") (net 2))
 (segment (start 108.1071 79.217894) (end 110.349994 76.975) (width 0.25) (layer "B.Cu") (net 2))
 (segment (start 90.875 75) (end 91 75) (width 0.25) (layer "B.Cu") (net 5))
 (segment (start 89.625001 86.05) (end 87.4 83.824999) (width 0.25) (layer "B.Cu") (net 5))
 (segment (start 87.4 83.824999) (end 87.4 78.475) (width 0.25) (layer "B.Cu") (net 5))
 (segment (start 87.4 78.475) (end 90.875 75) (width 0.25) (layer "B.Cu") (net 5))
 (segment (start 91.625001 86.05) (end 91.625001 78.125001) (width 0.25) (layer "B.Cu") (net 6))
 (segment (start 91.625001 78.125001) (end 91 77.5) (width 0.25) (layer "B.Cu") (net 6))
 (segment (start 87.625001 86.05) (end 86.775 85.199999) (width 0.25) (layer "B.Cu") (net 4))
 (segment (start 86.775 85.199999) (end 86.775 76.725) (width 0.25) (layer "B.Cu") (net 4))
 (segment (start 86.775 76.725) (end 91 72.5) (width 0.25) (layer "B.Cu") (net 4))
 (segment (start 108.349994 88.925) (end 107.5071 88.082106) (width 0.25) (layer "B.Cu") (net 1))
 (segment (start 107.5071 88.082106) (end 107.5071 74.737894) (width 0.25) (layer "B.Cu") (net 1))
 (segment (start 107.5071 74.737894) (end 110.349994 71.895) (width 0.25) (layer "B.Cu") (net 1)))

